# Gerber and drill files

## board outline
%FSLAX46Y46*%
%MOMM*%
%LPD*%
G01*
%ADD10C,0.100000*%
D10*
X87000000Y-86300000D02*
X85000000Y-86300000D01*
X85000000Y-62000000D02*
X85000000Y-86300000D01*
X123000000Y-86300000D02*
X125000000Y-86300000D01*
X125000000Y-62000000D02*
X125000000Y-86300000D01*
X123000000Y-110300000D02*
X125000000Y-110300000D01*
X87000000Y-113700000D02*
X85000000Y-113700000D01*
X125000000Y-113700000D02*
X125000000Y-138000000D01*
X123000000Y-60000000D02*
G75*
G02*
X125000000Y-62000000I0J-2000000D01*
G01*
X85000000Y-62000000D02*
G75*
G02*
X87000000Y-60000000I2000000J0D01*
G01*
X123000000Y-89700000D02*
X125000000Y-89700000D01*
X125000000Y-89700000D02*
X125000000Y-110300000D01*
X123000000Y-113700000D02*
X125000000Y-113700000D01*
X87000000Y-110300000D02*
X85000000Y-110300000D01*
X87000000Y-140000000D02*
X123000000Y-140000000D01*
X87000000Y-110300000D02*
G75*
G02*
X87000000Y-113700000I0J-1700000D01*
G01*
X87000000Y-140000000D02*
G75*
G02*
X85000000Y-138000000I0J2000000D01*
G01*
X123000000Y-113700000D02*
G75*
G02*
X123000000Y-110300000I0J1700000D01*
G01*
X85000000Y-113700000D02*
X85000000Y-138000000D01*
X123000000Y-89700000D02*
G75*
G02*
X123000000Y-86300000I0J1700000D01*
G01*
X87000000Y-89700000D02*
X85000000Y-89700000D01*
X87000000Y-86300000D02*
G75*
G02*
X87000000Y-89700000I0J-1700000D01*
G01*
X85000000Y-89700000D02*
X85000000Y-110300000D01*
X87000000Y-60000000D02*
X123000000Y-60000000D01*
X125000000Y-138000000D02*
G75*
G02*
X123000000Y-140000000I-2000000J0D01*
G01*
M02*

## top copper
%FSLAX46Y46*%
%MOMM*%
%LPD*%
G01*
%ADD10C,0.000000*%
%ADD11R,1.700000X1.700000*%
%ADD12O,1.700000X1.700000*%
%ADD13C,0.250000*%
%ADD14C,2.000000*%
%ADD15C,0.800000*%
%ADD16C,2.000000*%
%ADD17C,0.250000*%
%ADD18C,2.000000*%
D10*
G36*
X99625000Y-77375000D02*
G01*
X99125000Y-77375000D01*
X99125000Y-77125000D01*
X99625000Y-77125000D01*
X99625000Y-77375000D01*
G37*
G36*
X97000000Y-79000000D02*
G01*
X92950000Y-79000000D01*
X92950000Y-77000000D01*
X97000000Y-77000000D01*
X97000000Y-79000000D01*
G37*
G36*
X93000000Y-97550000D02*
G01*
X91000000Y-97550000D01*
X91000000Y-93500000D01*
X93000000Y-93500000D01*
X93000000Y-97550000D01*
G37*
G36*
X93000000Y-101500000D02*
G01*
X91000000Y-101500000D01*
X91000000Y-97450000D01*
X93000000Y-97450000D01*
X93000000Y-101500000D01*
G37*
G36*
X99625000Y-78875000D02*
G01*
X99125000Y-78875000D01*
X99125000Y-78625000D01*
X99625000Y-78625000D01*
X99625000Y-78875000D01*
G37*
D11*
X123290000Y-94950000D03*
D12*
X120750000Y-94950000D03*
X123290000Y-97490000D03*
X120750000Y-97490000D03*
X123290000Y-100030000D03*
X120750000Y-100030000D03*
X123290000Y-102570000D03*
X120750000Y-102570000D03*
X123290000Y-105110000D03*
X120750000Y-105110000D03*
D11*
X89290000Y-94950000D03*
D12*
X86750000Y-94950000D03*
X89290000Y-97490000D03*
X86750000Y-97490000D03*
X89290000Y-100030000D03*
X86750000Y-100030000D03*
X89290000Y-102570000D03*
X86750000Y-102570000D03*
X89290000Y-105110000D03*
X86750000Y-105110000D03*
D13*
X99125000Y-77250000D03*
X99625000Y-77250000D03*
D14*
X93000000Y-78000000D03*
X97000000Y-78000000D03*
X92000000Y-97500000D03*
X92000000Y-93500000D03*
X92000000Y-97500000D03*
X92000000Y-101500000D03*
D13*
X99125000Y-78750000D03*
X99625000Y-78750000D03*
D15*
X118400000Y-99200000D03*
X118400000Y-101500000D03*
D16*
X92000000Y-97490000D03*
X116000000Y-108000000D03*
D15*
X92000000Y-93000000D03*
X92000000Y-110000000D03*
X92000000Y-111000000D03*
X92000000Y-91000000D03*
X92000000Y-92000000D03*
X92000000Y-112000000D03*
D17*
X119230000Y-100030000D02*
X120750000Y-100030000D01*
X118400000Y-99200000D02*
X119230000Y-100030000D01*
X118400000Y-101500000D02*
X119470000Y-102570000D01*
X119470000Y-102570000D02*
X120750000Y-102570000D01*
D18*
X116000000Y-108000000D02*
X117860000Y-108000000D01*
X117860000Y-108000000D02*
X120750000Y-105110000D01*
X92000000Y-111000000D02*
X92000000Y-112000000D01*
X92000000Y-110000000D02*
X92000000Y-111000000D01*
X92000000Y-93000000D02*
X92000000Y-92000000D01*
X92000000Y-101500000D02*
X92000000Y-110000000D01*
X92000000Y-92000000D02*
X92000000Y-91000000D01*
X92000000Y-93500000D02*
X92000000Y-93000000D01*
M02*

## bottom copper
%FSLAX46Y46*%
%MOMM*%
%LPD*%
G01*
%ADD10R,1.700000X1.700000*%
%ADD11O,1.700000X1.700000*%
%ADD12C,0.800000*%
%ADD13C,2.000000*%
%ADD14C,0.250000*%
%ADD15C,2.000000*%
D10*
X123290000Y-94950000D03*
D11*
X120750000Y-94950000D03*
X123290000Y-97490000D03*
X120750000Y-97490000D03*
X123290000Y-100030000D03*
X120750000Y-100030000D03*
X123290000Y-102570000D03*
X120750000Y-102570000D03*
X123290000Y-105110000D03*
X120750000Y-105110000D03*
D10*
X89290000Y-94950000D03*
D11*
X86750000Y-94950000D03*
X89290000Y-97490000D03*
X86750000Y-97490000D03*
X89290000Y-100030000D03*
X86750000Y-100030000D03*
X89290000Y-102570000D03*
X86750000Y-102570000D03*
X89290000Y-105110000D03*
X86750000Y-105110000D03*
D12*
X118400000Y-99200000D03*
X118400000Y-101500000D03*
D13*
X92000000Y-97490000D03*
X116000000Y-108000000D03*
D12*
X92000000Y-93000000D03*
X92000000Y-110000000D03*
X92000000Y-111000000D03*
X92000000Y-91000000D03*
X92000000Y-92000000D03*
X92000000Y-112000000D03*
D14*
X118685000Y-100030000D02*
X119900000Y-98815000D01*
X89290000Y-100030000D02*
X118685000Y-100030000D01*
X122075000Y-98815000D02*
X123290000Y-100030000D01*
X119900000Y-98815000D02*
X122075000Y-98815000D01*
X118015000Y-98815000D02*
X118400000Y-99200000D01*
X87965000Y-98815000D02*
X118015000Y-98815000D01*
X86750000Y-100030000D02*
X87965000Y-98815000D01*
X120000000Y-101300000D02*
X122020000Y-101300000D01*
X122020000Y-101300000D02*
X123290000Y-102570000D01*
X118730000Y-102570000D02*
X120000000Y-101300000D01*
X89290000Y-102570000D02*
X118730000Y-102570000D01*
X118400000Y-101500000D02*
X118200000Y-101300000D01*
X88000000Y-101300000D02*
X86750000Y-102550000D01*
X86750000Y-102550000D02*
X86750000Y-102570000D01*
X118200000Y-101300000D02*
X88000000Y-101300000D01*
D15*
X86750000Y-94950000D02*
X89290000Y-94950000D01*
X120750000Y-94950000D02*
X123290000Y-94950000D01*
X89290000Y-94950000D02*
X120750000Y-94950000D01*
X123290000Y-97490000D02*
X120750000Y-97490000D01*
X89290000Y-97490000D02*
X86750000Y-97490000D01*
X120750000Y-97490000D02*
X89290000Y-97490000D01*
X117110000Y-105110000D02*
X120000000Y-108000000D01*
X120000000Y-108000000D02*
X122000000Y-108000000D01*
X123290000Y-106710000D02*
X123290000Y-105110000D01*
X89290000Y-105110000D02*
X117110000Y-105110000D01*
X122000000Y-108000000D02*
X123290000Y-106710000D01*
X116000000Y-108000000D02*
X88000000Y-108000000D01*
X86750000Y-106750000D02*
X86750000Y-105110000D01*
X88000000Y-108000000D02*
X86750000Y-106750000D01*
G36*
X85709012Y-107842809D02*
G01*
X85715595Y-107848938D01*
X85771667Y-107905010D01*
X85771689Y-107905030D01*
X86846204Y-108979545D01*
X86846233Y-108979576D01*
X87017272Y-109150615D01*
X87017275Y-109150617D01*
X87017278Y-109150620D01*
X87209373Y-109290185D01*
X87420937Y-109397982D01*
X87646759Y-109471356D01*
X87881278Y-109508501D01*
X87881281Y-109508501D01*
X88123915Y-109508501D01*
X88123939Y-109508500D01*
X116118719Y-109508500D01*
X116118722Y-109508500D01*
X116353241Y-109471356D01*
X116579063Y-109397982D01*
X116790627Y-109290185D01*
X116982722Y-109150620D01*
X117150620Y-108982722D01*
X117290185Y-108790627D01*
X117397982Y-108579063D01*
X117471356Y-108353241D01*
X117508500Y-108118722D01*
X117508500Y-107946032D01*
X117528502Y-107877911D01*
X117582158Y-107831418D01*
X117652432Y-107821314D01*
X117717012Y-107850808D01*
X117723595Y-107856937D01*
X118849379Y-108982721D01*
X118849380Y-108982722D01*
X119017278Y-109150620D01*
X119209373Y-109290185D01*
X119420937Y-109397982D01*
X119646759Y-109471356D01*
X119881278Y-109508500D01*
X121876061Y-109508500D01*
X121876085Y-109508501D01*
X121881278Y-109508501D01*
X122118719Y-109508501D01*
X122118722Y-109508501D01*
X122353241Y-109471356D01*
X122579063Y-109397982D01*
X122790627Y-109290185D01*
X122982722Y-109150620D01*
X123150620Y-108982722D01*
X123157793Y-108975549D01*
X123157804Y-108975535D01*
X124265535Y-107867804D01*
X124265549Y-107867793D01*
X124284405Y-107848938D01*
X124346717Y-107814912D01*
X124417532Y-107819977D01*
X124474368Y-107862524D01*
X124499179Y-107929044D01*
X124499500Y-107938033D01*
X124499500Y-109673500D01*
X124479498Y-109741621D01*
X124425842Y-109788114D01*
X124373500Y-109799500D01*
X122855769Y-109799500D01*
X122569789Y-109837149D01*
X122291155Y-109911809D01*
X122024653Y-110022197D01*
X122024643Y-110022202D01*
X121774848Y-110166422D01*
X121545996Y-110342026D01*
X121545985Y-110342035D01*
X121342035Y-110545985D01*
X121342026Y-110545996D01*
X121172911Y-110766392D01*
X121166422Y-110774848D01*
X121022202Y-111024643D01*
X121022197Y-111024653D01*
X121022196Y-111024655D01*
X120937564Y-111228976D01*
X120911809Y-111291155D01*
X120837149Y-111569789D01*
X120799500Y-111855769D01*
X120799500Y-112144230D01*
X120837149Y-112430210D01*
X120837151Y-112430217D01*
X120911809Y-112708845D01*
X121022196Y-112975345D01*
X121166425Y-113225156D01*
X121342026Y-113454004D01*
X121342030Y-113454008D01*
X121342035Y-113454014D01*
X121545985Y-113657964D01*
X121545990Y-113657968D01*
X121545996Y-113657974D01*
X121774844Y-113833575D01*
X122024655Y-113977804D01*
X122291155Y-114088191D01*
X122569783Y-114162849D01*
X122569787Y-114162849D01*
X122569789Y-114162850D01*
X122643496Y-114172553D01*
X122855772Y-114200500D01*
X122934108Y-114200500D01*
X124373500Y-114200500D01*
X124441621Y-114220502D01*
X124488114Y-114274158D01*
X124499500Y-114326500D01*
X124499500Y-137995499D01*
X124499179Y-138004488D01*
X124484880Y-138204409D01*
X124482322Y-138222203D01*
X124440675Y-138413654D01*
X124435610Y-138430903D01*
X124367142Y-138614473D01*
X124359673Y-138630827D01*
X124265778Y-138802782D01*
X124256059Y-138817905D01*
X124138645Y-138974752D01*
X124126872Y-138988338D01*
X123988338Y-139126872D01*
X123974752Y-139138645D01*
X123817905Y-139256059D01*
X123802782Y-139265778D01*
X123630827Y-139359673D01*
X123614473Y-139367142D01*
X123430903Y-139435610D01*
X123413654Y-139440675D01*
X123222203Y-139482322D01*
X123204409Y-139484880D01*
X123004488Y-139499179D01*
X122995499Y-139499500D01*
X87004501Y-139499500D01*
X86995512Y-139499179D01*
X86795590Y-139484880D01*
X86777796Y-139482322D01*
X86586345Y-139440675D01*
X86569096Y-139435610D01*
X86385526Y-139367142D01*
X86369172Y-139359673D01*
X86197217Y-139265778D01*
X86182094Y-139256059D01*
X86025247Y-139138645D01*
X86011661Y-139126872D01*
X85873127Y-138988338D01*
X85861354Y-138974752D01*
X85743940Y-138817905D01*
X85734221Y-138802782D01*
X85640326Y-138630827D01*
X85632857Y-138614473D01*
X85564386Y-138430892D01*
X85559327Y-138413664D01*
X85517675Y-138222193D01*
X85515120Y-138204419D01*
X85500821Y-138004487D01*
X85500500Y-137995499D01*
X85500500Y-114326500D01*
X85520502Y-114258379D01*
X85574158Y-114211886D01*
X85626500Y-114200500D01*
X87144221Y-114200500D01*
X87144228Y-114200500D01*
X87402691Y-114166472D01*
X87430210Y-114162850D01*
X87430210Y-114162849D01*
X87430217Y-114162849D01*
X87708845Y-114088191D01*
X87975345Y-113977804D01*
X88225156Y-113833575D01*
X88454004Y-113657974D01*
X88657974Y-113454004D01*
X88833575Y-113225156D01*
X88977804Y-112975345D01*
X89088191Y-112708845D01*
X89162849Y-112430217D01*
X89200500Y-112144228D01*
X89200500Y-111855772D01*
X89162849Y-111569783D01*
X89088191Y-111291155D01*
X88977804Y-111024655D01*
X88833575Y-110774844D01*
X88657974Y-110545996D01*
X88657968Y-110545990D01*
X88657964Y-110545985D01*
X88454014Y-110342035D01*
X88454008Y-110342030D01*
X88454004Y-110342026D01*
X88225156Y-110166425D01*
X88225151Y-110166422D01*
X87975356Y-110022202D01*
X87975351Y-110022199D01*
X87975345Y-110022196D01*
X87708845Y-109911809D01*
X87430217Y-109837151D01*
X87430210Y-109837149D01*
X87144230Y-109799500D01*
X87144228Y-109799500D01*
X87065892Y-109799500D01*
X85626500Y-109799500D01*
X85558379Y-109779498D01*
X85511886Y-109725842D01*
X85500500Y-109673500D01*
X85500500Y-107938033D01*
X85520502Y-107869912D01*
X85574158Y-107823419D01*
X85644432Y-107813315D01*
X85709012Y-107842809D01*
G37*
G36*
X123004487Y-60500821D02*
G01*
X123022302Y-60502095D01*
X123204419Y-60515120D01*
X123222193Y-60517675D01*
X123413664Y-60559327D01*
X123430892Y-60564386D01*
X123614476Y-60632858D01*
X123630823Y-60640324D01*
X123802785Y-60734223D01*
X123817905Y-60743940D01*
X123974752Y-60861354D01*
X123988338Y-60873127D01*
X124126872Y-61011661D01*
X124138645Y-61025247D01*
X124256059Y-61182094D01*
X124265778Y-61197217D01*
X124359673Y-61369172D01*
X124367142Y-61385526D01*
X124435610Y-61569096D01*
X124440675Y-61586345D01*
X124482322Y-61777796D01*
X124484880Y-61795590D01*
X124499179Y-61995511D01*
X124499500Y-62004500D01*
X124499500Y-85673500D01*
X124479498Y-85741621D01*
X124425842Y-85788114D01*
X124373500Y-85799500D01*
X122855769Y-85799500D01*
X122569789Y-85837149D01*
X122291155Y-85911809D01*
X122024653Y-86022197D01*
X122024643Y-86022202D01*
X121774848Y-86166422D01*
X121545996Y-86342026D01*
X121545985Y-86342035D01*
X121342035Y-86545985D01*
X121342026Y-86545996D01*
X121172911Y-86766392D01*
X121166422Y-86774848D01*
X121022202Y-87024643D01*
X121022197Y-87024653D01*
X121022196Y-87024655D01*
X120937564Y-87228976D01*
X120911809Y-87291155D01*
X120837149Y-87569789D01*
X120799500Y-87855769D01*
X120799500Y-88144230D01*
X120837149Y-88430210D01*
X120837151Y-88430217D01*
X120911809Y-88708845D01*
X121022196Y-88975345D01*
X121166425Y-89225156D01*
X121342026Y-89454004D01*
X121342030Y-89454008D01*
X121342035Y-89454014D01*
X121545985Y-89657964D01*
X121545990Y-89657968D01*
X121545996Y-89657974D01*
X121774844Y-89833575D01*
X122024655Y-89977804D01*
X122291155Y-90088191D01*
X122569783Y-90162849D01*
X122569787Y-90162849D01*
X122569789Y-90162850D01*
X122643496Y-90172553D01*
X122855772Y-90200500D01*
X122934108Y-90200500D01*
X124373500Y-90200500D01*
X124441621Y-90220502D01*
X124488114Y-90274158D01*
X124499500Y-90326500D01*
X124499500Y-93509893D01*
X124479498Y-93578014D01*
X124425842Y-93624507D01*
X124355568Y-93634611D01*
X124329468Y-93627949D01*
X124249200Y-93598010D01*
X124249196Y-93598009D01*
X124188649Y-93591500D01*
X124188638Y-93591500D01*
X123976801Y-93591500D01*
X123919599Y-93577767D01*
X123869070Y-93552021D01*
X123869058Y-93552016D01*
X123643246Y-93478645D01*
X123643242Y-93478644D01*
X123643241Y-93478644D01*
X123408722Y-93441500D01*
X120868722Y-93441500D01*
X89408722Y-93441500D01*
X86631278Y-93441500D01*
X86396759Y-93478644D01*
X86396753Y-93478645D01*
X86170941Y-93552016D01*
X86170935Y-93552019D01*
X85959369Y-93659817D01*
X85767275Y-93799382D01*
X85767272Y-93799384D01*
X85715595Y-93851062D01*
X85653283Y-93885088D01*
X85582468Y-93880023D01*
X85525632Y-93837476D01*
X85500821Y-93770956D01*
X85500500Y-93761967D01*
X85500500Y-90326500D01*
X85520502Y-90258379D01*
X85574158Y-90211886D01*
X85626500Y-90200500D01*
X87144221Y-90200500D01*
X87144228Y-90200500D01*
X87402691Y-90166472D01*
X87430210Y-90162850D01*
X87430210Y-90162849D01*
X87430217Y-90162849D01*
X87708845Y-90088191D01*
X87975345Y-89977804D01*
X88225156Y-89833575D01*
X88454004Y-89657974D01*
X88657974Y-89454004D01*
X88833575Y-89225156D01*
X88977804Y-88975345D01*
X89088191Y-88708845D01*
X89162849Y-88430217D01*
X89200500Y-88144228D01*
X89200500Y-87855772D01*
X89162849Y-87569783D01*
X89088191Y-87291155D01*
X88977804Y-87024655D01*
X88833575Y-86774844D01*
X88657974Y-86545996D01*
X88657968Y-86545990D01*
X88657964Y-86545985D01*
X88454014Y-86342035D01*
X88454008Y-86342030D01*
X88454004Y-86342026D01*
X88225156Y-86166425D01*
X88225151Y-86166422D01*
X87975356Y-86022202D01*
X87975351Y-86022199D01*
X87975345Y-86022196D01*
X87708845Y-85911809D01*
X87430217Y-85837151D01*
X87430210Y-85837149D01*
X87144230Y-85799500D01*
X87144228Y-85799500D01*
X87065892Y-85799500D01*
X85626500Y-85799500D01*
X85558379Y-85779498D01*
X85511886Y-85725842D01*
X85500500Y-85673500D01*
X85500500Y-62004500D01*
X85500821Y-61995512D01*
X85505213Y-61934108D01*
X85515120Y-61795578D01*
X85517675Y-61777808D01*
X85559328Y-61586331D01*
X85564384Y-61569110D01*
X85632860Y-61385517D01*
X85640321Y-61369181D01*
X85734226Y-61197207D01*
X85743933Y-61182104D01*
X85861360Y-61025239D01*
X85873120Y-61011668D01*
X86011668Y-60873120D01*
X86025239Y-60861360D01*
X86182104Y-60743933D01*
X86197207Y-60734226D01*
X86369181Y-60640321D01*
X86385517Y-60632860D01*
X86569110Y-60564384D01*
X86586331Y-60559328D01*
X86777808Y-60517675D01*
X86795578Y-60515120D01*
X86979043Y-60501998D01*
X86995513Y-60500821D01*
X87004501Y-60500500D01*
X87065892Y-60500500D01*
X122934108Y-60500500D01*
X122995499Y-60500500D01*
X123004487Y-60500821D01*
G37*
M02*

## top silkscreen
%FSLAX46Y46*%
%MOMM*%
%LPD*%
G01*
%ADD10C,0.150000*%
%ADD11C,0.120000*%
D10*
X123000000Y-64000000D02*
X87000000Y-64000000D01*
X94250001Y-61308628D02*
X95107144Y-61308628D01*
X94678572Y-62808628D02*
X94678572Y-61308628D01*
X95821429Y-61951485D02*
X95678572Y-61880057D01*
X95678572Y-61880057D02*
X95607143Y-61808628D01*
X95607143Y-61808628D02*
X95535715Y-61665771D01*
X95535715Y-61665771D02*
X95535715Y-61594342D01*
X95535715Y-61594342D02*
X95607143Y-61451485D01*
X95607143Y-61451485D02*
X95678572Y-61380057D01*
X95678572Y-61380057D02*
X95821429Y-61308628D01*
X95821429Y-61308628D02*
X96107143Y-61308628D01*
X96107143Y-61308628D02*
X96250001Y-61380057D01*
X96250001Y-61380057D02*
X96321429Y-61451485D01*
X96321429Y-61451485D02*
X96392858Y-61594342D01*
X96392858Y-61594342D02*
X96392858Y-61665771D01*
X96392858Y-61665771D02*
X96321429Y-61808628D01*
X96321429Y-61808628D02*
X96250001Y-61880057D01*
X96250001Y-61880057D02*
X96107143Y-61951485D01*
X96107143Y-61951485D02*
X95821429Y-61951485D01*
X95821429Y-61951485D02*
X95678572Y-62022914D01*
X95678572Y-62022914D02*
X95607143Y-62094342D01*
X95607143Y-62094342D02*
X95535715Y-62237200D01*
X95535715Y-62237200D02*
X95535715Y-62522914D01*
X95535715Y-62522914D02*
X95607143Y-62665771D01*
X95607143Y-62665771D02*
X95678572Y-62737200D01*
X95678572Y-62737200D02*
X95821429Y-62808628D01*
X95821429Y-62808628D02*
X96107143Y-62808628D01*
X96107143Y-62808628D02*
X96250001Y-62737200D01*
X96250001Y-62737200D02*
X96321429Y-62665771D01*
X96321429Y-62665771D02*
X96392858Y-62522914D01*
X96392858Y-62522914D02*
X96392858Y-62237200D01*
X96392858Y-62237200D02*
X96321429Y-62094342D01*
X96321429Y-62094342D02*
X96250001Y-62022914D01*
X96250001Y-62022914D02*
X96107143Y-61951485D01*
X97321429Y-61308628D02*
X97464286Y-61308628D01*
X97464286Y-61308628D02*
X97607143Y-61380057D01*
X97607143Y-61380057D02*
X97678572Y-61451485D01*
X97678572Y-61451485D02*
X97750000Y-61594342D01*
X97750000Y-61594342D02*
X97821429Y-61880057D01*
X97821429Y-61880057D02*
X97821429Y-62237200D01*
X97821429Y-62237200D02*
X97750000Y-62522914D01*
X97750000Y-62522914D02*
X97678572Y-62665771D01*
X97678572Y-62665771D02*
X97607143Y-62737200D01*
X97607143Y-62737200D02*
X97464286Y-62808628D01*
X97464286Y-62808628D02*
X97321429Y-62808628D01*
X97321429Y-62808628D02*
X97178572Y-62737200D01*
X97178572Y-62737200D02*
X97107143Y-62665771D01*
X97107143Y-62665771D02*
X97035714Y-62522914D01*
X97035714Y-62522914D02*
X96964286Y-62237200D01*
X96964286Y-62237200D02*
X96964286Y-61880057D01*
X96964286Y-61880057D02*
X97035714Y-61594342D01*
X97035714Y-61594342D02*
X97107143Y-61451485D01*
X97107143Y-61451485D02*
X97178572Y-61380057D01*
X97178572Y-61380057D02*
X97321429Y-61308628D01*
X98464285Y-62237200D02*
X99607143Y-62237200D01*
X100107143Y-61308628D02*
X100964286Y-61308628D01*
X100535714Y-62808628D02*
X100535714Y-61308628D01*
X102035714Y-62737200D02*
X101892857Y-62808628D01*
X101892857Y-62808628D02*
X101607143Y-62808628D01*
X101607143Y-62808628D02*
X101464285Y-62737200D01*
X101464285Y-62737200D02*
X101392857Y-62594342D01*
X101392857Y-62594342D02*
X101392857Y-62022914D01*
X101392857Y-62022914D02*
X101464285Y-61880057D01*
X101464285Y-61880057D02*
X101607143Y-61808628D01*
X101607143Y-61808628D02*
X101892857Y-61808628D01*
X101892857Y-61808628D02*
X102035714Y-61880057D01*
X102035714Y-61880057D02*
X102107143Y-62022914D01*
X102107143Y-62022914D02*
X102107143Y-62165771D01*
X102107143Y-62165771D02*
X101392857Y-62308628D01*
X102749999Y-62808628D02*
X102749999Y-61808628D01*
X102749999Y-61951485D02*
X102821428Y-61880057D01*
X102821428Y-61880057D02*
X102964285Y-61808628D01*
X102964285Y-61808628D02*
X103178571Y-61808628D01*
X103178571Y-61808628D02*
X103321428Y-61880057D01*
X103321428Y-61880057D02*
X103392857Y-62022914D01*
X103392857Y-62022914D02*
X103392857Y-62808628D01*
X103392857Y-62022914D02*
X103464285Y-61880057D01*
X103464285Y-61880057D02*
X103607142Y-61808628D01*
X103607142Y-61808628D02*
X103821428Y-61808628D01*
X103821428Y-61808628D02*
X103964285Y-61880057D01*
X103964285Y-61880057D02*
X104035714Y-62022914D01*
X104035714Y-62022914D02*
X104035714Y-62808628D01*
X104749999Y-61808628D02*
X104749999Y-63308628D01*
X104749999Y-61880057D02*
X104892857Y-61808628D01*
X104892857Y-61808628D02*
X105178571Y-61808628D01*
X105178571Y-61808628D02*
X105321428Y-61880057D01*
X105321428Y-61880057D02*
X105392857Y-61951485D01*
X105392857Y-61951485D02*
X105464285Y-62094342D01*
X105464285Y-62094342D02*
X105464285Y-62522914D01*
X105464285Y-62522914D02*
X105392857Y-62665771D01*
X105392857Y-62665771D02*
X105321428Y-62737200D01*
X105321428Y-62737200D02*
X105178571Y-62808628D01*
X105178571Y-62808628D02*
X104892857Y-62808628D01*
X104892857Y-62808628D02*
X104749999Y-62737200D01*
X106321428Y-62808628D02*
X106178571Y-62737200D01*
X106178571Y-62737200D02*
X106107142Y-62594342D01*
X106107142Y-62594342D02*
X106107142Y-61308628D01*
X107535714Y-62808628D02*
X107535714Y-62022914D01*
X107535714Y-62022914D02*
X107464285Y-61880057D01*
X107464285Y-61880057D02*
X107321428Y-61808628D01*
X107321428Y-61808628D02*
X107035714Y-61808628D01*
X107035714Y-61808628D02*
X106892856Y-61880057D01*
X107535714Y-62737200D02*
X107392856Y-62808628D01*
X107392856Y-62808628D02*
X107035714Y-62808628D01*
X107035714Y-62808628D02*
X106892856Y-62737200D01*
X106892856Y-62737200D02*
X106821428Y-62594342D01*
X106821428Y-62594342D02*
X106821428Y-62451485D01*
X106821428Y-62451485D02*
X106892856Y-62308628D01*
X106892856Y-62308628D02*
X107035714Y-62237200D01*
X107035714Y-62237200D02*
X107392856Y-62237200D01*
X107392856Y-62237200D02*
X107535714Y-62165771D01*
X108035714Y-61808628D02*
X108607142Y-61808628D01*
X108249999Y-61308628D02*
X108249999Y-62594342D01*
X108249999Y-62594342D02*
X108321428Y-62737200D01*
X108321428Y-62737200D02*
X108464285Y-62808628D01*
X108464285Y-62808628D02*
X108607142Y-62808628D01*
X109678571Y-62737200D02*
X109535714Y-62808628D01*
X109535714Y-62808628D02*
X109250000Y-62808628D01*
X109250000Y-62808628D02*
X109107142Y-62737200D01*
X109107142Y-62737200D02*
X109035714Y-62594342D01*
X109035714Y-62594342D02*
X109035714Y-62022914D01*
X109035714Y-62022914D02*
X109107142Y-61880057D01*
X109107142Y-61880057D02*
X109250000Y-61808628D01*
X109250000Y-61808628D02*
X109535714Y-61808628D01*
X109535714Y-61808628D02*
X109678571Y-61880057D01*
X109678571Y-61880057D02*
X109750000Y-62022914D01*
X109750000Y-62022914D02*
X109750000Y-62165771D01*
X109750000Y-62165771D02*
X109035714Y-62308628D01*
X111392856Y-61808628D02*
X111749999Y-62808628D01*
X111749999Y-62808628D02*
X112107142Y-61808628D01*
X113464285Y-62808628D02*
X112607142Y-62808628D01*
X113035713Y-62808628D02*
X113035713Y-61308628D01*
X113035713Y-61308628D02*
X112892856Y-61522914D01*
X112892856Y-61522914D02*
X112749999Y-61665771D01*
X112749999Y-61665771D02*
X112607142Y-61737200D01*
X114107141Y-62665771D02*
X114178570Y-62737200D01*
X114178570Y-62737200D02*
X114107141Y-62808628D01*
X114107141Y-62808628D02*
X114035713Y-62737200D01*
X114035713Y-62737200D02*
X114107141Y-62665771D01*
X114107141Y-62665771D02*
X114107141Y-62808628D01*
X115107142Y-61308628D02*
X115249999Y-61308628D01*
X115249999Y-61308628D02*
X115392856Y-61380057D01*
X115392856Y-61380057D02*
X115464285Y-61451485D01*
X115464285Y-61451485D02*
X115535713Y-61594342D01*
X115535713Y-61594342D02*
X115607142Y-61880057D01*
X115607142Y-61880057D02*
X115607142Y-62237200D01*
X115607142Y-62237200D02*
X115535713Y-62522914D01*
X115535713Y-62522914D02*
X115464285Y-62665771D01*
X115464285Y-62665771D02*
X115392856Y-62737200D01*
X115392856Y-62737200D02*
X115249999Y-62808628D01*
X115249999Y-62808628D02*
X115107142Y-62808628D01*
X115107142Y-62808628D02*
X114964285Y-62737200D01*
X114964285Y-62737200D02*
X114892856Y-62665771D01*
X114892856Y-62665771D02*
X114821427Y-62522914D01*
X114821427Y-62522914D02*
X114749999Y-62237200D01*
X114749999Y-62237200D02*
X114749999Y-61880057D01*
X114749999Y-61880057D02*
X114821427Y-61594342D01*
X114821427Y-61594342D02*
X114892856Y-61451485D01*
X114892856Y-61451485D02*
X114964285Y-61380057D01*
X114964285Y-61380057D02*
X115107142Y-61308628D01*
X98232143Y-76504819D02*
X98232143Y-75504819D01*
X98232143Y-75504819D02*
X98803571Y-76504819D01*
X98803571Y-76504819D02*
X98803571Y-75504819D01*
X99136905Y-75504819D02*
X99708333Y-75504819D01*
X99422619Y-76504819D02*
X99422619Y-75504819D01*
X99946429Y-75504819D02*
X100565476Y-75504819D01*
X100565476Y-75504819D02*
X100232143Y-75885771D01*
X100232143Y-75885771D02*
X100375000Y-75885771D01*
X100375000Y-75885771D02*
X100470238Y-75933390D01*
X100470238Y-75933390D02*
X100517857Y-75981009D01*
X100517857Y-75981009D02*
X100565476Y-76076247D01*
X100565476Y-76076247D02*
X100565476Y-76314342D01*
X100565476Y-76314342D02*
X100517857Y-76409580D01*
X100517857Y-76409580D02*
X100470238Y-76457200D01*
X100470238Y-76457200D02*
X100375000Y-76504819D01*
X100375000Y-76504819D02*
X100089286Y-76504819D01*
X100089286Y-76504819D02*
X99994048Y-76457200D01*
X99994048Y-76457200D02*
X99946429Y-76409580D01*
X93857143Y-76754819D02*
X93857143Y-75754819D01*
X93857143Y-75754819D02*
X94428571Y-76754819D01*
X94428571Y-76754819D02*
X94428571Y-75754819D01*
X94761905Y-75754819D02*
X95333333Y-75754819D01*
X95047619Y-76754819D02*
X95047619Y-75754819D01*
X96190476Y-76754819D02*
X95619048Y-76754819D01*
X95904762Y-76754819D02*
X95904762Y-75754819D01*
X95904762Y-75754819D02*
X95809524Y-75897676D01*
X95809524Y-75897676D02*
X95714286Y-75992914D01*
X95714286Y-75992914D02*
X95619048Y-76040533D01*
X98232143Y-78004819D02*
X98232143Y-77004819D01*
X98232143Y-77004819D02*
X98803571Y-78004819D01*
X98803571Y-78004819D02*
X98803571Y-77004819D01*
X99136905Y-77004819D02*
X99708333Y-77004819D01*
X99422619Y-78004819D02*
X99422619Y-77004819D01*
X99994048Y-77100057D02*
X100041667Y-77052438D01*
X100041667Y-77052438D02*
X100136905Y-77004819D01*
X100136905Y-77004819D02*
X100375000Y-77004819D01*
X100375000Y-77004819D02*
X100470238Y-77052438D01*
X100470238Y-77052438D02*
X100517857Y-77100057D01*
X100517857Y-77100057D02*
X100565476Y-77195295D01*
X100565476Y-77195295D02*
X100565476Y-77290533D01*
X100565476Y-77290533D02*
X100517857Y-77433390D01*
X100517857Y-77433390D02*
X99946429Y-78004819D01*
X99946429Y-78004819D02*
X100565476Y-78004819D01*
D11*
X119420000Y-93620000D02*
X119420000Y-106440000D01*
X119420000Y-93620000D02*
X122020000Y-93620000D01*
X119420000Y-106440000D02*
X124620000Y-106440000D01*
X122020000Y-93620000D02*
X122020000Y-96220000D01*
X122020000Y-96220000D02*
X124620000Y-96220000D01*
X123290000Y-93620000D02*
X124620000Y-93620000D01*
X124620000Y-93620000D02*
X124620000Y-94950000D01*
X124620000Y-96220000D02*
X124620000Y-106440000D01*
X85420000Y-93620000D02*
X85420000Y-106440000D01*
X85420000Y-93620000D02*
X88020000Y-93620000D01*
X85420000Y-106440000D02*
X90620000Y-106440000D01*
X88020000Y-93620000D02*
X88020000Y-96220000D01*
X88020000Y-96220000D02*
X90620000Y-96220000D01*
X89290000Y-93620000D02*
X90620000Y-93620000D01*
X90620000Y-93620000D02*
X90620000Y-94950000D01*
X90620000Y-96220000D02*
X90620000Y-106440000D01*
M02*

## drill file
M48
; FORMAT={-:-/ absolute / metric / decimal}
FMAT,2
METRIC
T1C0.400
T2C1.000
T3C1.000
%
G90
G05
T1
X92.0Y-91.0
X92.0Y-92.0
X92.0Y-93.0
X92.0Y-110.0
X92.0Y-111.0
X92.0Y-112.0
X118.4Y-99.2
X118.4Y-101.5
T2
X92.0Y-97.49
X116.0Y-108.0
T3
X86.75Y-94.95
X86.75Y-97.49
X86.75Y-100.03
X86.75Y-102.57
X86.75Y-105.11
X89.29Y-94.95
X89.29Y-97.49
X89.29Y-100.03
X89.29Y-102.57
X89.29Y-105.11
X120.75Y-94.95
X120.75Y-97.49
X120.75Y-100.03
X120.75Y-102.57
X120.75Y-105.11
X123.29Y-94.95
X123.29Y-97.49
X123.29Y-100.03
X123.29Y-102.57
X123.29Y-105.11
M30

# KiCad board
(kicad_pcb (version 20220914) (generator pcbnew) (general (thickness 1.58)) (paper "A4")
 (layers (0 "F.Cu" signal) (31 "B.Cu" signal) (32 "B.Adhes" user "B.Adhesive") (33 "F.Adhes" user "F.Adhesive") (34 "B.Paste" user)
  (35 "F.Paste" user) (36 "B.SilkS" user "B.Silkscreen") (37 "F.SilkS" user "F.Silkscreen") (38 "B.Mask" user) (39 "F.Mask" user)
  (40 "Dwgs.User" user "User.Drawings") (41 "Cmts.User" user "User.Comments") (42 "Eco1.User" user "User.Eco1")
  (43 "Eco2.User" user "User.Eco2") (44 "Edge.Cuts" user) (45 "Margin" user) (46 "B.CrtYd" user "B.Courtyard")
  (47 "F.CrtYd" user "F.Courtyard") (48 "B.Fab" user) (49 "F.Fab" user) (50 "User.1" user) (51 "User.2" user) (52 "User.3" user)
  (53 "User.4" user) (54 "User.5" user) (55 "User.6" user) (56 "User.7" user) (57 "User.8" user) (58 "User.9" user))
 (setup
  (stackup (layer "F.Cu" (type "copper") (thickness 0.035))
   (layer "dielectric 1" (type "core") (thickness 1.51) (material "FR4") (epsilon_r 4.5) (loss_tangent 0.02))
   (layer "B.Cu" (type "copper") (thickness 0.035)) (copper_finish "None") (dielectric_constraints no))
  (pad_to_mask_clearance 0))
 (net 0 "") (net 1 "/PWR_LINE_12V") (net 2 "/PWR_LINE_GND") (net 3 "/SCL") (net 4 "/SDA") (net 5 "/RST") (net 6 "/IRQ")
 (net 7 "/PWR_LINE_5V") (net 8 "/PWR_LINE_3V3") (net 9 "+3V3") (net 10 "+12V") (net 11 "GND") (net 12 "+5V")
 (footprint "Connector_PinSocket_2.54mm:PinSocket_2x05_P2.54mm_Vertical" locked (layer "F.Cu") (at 123.29 94.95)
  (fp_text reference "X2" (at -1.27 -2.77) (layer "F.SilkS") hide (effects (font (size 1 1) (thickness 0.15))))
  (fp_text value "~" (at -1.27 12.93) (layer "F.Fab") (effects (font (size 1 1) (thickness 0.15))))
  (fp_line (start -3.87 -1.33) (end -3.87 11.49) (stroke (width 0.12) (type solid)) (layer "F.SilkS"))
  (fp_line (start -3.87 -1.33) (end -1.27 -1.33) (stroke (width 0.12) (type solid)) (layer "F.SilkS"))
  (fp_line (start -3.87 11.49) (end 1.33 11.49) (stroke (width 0.12) (type solid)) (layer "F.SilkS"))
  (fp_line (start -1.27 -1.33) (end -1.27 1.27) (stroke (width 0.12) (type solid)) (layer "F.SilkS"))
  (fp_line (start -1.27 1.27) (end 1.33 1.27) (stroke (width 0.12) (type solid)) (layer "F.SilkS"))
  (fp_line (start 0 -1.33) (end 1.33 -1.33) (stroke (width 0.12) (type solid)) (layer "F.SilkS"))
  (fp_line (start 1.33 -1.33) (end 1.33 0) (stroke (width 0.12) (type solid)) (layer "F.SilkS"))
  (fp_line (start 1.33 1.27) (end 1.33 11.49) (stroke (width 0.12) (type solid)) (layer "F.SilkS"))
  (pad "1" thru_hole rect locked (at 0 0) (size 1.7 1.7) (drill 1) (layers *.Cu *.Mask) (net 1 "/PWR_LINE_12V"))
  (pad "2" thru_hole oval locked (at -2.54 0) (size 1.7 1.7) (drill 1) (layers *.Cu *.Mask) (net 1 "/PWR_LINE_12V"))
  (pad "3" thru_hole oval locked (at 0 2.54) (size 1.7 1.7) (drill 1) (layers *.Cu *.Mask) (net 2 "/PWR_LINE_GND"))
  (pad "4" thru_hole oval locked (at -2.54 2.54) (size 1.7 1.7) (drill 1) (layers *.Cu *.Mask) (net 2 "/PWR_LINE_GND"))
  (pad "5" thru_hole oval locked (at 0 5.08) (size 1.7 1.7) (drill 1) (layers *.Cu *.Mask) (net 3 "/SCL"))
  (pad "6" thru_hole oval locked (at -2.54 5.08) (size 1.7 1.7) (drill 1) (layers *.Cu *.Mask) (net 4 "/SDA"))
  (pad "7" thru_hole oval locked (at 0 7.62) (size 1.7 1.7) (drill 1) (layers *.Cu *.Mask) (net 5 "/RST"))
  (pad "8" thru_hole oval locked (at -2.54 7.62) (size 1.7 1.7) (drill 1) (layers *.Cu *.Mask) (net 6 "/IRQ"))
  (pad "9" thru_hole oval locked (at 0 10.16) (size 1.7 1.7) (drill 1) (layers *.Cu *.Mask) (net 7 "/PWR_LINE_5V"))
  (pad "10" thru_hole oval locked (at -2.54 10.16) (size 1.7 1.7) (drill 1) (layers *.Cu *.Mask) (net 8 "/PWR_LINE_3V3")))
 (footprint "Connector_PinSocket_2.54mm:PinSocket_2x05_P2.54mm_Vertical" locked (layer "F.Cu") (at 89.29 94.95)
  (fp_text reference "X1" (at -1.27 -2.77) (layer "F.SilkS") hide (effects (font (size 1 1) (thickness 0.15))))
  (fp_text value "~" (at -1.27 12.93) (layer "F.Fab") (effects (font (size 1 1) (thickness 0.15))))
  (fp_line (start -3.87 -1.33) (end -3.87 11.49) (stroke (width 0.12) (type solid)) (layer "F.SilkS"))
  (fp_line (start -3.87 -1.33) (end -1.27 -1.33) (stroke (width 0.12) (type solid)) (layer "F.SilkS"))
  (fp_line (start -3.87 11.49) (end 1.33 11.49) (stroke (width 0.12) (type solid)) (layer "F.SilkS"))
  (fp_line (start -1.27 -1.33) (end -1.27 1.27) (stroke (width 0.12) (type solid)) (layer "F.SilkS"))
  (fp_line (start -1.27 1.27) (end 1.33 1.27) (stroke (width 0.12) (type solid)) (layer "F.SilkS"))
  (fp_line (start 0 -1.33) (end 1.33 -1.33) (stroke (width 0.12) (type solid)) (layer "F.SilkS"))
  (fp_line (start 1.33 -1.33) (end 1.33 0) (stroke (width 0.12) (type solid)) (layer "F.SilkS"))
  (fp_line (start 1.33 1.27) (end 1.33 11.49) (stroke (width 0.12) (type solid)) (layer "F.SilkS"))
  (pad "1" thru_hole rect locked (at 0 0) (size 1.7 1.7) (drill 1) (layers *.Cu *.Mask) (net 1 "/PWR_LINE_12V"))
  (pad "2" thru_hole oval locked (at -2.54 0) (size 1.7 1.7) (drill 1) (layers *.Cu *.Mask) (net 1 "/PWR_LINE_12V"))
  (pad "3" thru_hole oval locked (at 0 2.54) (size 1.7 1.7) (drill 1) (layers *.Cu *.Mask) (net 2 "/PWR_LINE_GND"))
  (pad "4" thru_hole oval locked (at -2.54 2.54) (size 1.7 1.7) (drill 1) (layers *.Cu *.Mask) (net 2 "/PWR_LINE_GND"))
  (pad "5" thru_hole oval locked (at 0 5.08) (size 1.7 1.7) (drill 1) (layers *.Cu *.Mask) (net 3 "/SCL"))
  (pad "6" thru_hole oval locked (at -2.54 5.08) (size 1.7 1.7) (drill 1) (layers *.Cu *.Mask) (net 4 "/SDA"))
  (pad "7" thru_hole oval locked (at 0 7.62) (size 1.7 1.7) (drill 1) (layers *.Cu *.Mask) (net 5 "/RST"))
  (pad "8" thru_hole oval locked (at -2.54 7.62) (size 1.7 1.7) (drill 1) (layers *.Cu *.Mask) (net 6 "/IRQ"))
  (pad "9" thru_hole oval locked (at 0 10.16) (size 1.7 1.7) (drill 1) (layers *.Cu *.Mask) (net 7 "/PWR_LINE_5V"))
  (pad "10" thru_hole oval locked (at -2.54 10.16) (size 1.7 1.7) (drill 1) (layers *.Cu *.Mask) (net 8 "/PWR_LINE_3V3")))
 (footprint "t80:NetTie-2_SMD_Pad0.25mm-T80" (layer "F.Cu") (at 99.375 77.25) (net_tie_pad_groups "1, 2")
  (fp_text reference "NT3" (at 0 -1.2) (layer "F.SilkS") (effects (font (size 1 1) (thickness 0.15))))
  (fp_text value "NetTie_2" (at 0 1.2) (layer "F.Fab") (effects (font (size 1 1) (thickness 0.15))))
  (fp_poly
   (pts (xy -0.25 -0.125) (xy 0.25 -0.125) (xy 0.25 0.125) (xy -0.25 0.125)) (stroke (width 0) (type solid)) (fill solid) (layer "F.Cu"))
  (pad "1" smd circle (at -0.25 0) (size 0.25 0.25) (layers "F.Cu") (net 8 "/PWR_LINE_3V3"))
  (pad "2" smd circle (at 0.25 0) (size 0.25 0.25) (layers "F.Cu") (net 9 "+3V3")))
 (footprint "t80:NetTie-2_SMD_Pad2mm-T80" (layer "F.Cu") (at 95 78) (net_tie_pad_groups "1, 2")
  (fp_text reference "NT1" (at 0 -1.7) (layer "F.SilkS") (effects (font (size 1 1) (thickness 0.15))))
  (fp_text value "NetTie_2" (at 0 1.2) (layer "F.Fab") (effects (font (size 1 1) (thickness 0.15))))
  (fp_poly (pts (xy -2.05 -1) (xy 2 -1) (xy 2 1) (xy -2.05 1)) (stroke (width 0) (type solid)) (fill solid) (layer "F.Cu"))
  (pad "1" smd circle (at -2 0) (size 2 2) (layers "F.Cu") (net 1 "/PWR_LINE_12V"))
  (pad "2" smd circle (at 2 0) (size 2 2) (layers "F.Cu") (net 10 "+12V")))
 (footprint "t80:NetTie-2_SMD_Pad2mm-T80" (layer "F.Cu") (at 92 95.5 90) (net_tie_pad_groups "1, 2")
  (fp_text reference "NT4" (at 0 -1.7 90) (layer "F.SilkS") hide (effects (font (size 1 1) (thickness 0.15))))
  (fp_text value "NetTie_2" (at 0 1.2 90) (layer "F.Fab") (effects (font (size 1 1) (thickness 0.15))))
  (fp_poly (pts (xy -2.05 -1) (xy 2 -1) (xy 2 1) (xy -2.05 1)) (stroke (width 0) (type solid)) (fill solid) (layer "F.Cu"))
  (pad "1" smd circle (at -2 0 90) (size 2 2) (layers "F.Cu") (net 2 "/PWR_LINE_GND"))
  (pad "2" smd circle (at 2 0 90) (size 2 2) (layers "F.Cu") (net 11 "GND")))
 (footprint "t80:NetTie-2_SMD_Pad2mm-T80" (layer "F.Cu") (at 92 99.5 -90) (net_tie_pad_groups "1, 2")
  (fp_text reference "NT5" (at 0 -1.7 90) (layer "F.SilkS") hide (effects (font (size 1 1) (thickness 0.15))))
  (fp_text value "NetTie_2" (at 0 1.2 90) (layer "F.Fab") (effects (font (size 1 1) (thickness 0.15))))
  (fp_poly (pts (xy -2.05 -1) (xy 2 -1) (xy 2 1) (xy -2.05 1)) (stroke (width 0) (type solid)) (fill solid) (layer "F.Cu"))
  (pad "1" smd circle (at -2 0 270) (size 2 2) (layers "F.Cu") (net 2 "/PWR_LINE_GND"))
  (pad "2" smd circle (at 2 0 270) (size 2 2) (layers "F.Cu") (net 11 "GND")))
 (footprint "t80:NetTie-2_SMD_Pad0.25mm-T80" (layer "F.Cu") (at 99.375 78.75) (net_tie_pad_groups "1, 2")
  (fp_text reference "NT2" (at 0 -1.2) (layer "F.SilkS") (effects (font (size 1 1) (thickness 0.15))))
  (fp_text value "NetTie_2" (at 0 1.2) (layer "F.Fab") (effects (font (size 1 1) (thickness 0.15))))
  (fp_poly
   (pts (xy -0.25 -0.125) (xy 0.25 -0.125) (xy 0.25 0.125) (xy -0.25 0.125)) (stroke (width 0) (type solid)) (fill solid) (layer "F.Cu"))
  (pad "1" smd circle (at -0.25 0) (size 0.25 0.25) (layers "F.Cu") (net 7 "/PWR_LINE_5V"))
  (pad "2" smd circle (at 0.25 0) (size 0.25 0.25) (layers "F.Cu") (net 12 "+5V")))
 (gr_line (start 123 64) (end 87 64) (stroke (width 0.15) (type default)) (layer "F.SilkS"))
 (gr_line (start 87 86.3) (end 85 86.3) (stroke (width 0.1) (type default)) (layer "Edge.Cuts"))
 (gr_line (start 85 62) (end 85 86.3) (stroke (width 0.1) (type default)) (layer "Edge.Cuts"))
 (gr_line (start 123 86.3) (end 125 86.3) (stroke (width 0.1) (type default)) (layer "Edge.Cuts"))
 (gr_line (start 125 62) (end 125 86.3) (stroke (width 0.1) (type default)) (layer "Edge.Cuts"))
 (gr_line (start 123 110.3) (end 125 110.3) (stroke (width 0.1) (type default)) (layer "Edge.Cuts"))
 (gr_line (start 87 113.7) (end 85 113.7) (stroke (width 0.1) (type default)) (layer "Edge.Cuts"))
 (gr_line (start 125 113.7) (end 125 138) (stroke (width 0.1) (type default)) (layer "Edge.Cuts"))
 (gr_arc (start 123 60) (mid 124.414214 60.585786) (end 125 62) (stroke (width 0.1) (type default)) (layer "Edge.Cuts"))
 (gr_arc (start 85 62) (mid 85.585786 60.585786) (end 87 60) (stroke (width 0.1) (type default)) (layer "Edge.Cuts"))
 (gr_line (start 123 89.7) (end 125 89.7) (stroke (width 0.1) (type default)) (layer "Edge.Cuts"))
 (gr_line (start 125 89.7) (end 125 110.3) (stroke (width 0.1) (type default)) (layer "Edge.Cuts"))
 (gr_line (start 123 113.7) (end 125 113.7) (stroke (width 0.1) (type default)) (layer "Edge.Cuts"))
 (gr_line (start 87 110.3) (end 85 110.3) (stroke (width 0.1) (type default)) (layer "Edge.Cuts"))
 (gr_line (start 87 140) (end 123 140) (stroke (width 0.1) (type default)) (layer "Edge.Cuts"))
 (gr_arc (start 87 110.3) (mid 88.7 112) (end 87 113.7) (stroke (width 0.1) (type default)) (layer "Edge.Cuts"))
 (gr_arc (start 87 140) (mid 85.585786 139.414214) (end 85 138) (stroke (width 0.1) (type default)) (layer "Edge.Cuts"))
 (gr_arc (start 123 113.7) (mid 121.3 112) (end 123 110.3) (stroke (width 0.1) (type default)) (layer "Edge.Cuts"))
 (gr_line (start 85 113.7) (end 85 138) (stroke (width 0.1) (type default)) (layer "Edge.Cuts"))
 (gr_arc (start 123 89.7) (mid 121.3 88) (end 123 86.3) (stroke (width 0.1) (type default)) (layer "Edge.Cuts"))
 (gr_line (start 87 89.7) (end 85 89.7) (stroke (width 0.1) (type default)) (layer "Edge.Cuts"))
 (gr_arc (start 87 86.3) (mid 88.7 88) (end 87 89.7) (stroke (width 0.1) (type default)) (layer "Edge.Cuts"))
 (gr_line (start 85 89.7) (end 85 110.3) (stroke (width 0.1) (type default)) (layer "Edge.Cuts"))
 (gr_line (start 87 60) (end 123 60) (stroke (width 0.1) (type default)) (layer "Edge.Cuts"))
 (gr_arc (start 125 138) (mid 124.414214 139.414214) (end 123 140) (stroke (width 0.1) (type default)) (layer "Edge.Cuts"))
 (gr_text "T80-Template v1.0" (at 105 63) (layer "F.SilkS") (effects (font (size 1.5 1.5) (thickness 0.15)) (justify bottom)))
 (segment (start 118.685 100.03) (end 119.9 98.815) (width 0.25) (layer "B.Cu") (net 3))
 (segment (start 89.29 100.03) (end 118.685 100.03) (width 0.25) (layer "B.Cu") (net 3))
 (segment (start 122.075 98.815) (end 123.29 100.03) (width 0.25) (layer "B.Cu") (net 3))
 (segment (start 119.9 98.815) (end 122.075 98.815) (width 0.25) (layer "B.Cu") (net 3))
 (segment (start 119.23 100.03) (end 120.75 100.03) (width 0.25) (layer "F.Cu") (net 4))
 (segment (start 118.4 99.2) (end 119.23 100.03) (width 0.25) (layer "F.Cu") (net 4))
 (via (at 118.4 99.2) (size 0.8) (drill 0.4) (layers "F.Cu" "B.Cu") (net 4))
 (segment (start 118.015 98.815) (end 118.4 99.2) (width 0.25) (layer "B.Cu") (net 4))
 (segment (start 87.965 98.815) (end 118.015 98.815) (width 0.25) (layer "B.Cu") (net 4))
 (segment (start 86.75 100.03) (end 87.965 98.815) (width 0.25) (layer "B.Cu") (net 4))
 (segment (start 120 101.3) (end 122.02 101.3) (width 0.25) (layer "B.Cu") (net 5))
 (segment (start 122.02 101.3) (end 123.29 102.57) (width 0.25) (layer "B.Cu") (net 5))
 (segment (start 118.73 102.57) (end 120 101.3) (width 0.25) (layer "B.Cu") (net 5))
 (segment (start 89.29 102.57) (end 118.73 102.57) (width 0.25) (layer "B.Cu") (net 5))
 (segment (start 118.4 101.5) (end 119.47 102.57) (width 0.25) (layer "F.Cu") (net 6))
 (segment (start 119.47 102.57) (end 120.75 102.57) (width 0.25) (layer "F.Cu") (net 6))
 (via (at 118.4 101.5) (size 0.8) (drill 0.4) (layers "F.Cu" "B.Cu") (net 6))
 (segment (start 118.4 101.5) (end 118.2 101.3) (width 0.25) (layer "B.Cu") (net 6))
 (segment (start 88 101.3) (end 86.75 102.55) (width 0.25) (layer "B.Cu") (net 6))
 (segment (start 86.75 102.55) (end 86.75 102.57) (width 0.25) (layer "B.Cu") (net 6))
 (segment (start 118.2 101.3) (end 88 101.3) (width 0.25) (layer "B.Cu") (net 6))
 (segment (start 86.75 94.95) (end 89.29 94.95) (width 2) (layer "B.Cu") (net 1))
 (segment (start 120.75 94.95) (end 123.29 94.95) (width 2) (layer "B.Cu") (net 1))
 (segment (start 89.29 94.95) (end 120.75 94.95) (width 2) (layer "B.Cu") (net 1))
 (via (at 92 97.49) (size 2) (drill 1) (layers "F.Cu" "B.Cu") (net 2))
 (segment (start 123.29 97.49) (end 120.75 97.49) (width 2) (layer "B.Cu") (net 2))
 (segment (start 89.29 97.49) (end 86.75 97.49) (width 2) (layer "B.Cu") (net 2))
 (segment (start 120.75 97.49) (end 89.29 97.49) (width 2) (layer "B.Cu") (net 2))
 (segment (start 117.11 105.11) (end 120 108) (width 2) (layer "B.Cu") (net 7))
 (segment (start 120 108) (end 122 108) (width 2) (layer "B.Cu") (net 7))
 (segment (start 123.29 106.71) (end 123.29 105.11) (width 2) (layer "B.Cu") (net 7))
 (segment (start 89.29 105.11) (end 117.11 105.11) (width 2) (layer "B.Cu") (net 7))
 (segment (start 122 108) (end 123.29 106.71) (width 2) (layer "B.Cu") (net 7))
 (segment (start 116 108) (end 117.86 108) (width 2) (layer "F.Cu") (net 8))
 (segment (start 117.86 108) (end 120.75 105.11) (width 2) (layer "F.Cu") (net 8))
 (via (at 116 108) (size 2) (drill 1) (layers "F.Cu" "B.Cu") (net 8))
 (segment (start 116 108) (end 88 108) (width 2) (layer "B.Cu") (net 8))
 (segment (start 86.75 106.75) (end 86.75 105.11) (width 2) (layer "B.Cu") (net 8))
 (segment (start 88 108) (end 86.75 106.75) (width 2) (layer "B.Cu") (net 8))
 (segment (start 92 111) (end 92 112) (width 2) (layer "F.Cu") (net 11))
 (segment (start 92 110) (end 92 111) (width 2) (layer "F.Cu") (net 11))
 (segment (start 92 93) (end 92 92) (width 2) (layer "F.Cu") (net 11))
 (segment (start 92 101.5) (end 92 110) (width 2) (layer "F.Cu") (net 11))
 (segment (start 92 92) (end 92 91) (width 2) (layer "F.Cu") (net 11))
 (segment (start 92 93.5) (end 92 93) (width 2) (layer "F.Cu") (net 11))
 (via (at 92 93) (size 0.8) (drill 0.4) (layers "F.Cu" "B.Cu") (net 11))
 (via (at 92 110) (size 0.8) (drill 0.4) (layers "F.Cu" "B.Cu") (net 11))
 (via (at 92 111) (size 0.8) (drill 0.4) (layers "F.Cu" "B.Cu") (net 11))
 (via (at 92 91) (size 0.8) (drill 0.4) (layers "F.Cu" "B.Cu") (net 11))
 (via (at 92 92) (size 0.8) (drill 0.4) (layers "F.Cu" "B.Cu") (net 11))
 (via (at 92 112) (size 0.8) (drill 0.4) (layers "F.Cu" "B.Cu") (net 11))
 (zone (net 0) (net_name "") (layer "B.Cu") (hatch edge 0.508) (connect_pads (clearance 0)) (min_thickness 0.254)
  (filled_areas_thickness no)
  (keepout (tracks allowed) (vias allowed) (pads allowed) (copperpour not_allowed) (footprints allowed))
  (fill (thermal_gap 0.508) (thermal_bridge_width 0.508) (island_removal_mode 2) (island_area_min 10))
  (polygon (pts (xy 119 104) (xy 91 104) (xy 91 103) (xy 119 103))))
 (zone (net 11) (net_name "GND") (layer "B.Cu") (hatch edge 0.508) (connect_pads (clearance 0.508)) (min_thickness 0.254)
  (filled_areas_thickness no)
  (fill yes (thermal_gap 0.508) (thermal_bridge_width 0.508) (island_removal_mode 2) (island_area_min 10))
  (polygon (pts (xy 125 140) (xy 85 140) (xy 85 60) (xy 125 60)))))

